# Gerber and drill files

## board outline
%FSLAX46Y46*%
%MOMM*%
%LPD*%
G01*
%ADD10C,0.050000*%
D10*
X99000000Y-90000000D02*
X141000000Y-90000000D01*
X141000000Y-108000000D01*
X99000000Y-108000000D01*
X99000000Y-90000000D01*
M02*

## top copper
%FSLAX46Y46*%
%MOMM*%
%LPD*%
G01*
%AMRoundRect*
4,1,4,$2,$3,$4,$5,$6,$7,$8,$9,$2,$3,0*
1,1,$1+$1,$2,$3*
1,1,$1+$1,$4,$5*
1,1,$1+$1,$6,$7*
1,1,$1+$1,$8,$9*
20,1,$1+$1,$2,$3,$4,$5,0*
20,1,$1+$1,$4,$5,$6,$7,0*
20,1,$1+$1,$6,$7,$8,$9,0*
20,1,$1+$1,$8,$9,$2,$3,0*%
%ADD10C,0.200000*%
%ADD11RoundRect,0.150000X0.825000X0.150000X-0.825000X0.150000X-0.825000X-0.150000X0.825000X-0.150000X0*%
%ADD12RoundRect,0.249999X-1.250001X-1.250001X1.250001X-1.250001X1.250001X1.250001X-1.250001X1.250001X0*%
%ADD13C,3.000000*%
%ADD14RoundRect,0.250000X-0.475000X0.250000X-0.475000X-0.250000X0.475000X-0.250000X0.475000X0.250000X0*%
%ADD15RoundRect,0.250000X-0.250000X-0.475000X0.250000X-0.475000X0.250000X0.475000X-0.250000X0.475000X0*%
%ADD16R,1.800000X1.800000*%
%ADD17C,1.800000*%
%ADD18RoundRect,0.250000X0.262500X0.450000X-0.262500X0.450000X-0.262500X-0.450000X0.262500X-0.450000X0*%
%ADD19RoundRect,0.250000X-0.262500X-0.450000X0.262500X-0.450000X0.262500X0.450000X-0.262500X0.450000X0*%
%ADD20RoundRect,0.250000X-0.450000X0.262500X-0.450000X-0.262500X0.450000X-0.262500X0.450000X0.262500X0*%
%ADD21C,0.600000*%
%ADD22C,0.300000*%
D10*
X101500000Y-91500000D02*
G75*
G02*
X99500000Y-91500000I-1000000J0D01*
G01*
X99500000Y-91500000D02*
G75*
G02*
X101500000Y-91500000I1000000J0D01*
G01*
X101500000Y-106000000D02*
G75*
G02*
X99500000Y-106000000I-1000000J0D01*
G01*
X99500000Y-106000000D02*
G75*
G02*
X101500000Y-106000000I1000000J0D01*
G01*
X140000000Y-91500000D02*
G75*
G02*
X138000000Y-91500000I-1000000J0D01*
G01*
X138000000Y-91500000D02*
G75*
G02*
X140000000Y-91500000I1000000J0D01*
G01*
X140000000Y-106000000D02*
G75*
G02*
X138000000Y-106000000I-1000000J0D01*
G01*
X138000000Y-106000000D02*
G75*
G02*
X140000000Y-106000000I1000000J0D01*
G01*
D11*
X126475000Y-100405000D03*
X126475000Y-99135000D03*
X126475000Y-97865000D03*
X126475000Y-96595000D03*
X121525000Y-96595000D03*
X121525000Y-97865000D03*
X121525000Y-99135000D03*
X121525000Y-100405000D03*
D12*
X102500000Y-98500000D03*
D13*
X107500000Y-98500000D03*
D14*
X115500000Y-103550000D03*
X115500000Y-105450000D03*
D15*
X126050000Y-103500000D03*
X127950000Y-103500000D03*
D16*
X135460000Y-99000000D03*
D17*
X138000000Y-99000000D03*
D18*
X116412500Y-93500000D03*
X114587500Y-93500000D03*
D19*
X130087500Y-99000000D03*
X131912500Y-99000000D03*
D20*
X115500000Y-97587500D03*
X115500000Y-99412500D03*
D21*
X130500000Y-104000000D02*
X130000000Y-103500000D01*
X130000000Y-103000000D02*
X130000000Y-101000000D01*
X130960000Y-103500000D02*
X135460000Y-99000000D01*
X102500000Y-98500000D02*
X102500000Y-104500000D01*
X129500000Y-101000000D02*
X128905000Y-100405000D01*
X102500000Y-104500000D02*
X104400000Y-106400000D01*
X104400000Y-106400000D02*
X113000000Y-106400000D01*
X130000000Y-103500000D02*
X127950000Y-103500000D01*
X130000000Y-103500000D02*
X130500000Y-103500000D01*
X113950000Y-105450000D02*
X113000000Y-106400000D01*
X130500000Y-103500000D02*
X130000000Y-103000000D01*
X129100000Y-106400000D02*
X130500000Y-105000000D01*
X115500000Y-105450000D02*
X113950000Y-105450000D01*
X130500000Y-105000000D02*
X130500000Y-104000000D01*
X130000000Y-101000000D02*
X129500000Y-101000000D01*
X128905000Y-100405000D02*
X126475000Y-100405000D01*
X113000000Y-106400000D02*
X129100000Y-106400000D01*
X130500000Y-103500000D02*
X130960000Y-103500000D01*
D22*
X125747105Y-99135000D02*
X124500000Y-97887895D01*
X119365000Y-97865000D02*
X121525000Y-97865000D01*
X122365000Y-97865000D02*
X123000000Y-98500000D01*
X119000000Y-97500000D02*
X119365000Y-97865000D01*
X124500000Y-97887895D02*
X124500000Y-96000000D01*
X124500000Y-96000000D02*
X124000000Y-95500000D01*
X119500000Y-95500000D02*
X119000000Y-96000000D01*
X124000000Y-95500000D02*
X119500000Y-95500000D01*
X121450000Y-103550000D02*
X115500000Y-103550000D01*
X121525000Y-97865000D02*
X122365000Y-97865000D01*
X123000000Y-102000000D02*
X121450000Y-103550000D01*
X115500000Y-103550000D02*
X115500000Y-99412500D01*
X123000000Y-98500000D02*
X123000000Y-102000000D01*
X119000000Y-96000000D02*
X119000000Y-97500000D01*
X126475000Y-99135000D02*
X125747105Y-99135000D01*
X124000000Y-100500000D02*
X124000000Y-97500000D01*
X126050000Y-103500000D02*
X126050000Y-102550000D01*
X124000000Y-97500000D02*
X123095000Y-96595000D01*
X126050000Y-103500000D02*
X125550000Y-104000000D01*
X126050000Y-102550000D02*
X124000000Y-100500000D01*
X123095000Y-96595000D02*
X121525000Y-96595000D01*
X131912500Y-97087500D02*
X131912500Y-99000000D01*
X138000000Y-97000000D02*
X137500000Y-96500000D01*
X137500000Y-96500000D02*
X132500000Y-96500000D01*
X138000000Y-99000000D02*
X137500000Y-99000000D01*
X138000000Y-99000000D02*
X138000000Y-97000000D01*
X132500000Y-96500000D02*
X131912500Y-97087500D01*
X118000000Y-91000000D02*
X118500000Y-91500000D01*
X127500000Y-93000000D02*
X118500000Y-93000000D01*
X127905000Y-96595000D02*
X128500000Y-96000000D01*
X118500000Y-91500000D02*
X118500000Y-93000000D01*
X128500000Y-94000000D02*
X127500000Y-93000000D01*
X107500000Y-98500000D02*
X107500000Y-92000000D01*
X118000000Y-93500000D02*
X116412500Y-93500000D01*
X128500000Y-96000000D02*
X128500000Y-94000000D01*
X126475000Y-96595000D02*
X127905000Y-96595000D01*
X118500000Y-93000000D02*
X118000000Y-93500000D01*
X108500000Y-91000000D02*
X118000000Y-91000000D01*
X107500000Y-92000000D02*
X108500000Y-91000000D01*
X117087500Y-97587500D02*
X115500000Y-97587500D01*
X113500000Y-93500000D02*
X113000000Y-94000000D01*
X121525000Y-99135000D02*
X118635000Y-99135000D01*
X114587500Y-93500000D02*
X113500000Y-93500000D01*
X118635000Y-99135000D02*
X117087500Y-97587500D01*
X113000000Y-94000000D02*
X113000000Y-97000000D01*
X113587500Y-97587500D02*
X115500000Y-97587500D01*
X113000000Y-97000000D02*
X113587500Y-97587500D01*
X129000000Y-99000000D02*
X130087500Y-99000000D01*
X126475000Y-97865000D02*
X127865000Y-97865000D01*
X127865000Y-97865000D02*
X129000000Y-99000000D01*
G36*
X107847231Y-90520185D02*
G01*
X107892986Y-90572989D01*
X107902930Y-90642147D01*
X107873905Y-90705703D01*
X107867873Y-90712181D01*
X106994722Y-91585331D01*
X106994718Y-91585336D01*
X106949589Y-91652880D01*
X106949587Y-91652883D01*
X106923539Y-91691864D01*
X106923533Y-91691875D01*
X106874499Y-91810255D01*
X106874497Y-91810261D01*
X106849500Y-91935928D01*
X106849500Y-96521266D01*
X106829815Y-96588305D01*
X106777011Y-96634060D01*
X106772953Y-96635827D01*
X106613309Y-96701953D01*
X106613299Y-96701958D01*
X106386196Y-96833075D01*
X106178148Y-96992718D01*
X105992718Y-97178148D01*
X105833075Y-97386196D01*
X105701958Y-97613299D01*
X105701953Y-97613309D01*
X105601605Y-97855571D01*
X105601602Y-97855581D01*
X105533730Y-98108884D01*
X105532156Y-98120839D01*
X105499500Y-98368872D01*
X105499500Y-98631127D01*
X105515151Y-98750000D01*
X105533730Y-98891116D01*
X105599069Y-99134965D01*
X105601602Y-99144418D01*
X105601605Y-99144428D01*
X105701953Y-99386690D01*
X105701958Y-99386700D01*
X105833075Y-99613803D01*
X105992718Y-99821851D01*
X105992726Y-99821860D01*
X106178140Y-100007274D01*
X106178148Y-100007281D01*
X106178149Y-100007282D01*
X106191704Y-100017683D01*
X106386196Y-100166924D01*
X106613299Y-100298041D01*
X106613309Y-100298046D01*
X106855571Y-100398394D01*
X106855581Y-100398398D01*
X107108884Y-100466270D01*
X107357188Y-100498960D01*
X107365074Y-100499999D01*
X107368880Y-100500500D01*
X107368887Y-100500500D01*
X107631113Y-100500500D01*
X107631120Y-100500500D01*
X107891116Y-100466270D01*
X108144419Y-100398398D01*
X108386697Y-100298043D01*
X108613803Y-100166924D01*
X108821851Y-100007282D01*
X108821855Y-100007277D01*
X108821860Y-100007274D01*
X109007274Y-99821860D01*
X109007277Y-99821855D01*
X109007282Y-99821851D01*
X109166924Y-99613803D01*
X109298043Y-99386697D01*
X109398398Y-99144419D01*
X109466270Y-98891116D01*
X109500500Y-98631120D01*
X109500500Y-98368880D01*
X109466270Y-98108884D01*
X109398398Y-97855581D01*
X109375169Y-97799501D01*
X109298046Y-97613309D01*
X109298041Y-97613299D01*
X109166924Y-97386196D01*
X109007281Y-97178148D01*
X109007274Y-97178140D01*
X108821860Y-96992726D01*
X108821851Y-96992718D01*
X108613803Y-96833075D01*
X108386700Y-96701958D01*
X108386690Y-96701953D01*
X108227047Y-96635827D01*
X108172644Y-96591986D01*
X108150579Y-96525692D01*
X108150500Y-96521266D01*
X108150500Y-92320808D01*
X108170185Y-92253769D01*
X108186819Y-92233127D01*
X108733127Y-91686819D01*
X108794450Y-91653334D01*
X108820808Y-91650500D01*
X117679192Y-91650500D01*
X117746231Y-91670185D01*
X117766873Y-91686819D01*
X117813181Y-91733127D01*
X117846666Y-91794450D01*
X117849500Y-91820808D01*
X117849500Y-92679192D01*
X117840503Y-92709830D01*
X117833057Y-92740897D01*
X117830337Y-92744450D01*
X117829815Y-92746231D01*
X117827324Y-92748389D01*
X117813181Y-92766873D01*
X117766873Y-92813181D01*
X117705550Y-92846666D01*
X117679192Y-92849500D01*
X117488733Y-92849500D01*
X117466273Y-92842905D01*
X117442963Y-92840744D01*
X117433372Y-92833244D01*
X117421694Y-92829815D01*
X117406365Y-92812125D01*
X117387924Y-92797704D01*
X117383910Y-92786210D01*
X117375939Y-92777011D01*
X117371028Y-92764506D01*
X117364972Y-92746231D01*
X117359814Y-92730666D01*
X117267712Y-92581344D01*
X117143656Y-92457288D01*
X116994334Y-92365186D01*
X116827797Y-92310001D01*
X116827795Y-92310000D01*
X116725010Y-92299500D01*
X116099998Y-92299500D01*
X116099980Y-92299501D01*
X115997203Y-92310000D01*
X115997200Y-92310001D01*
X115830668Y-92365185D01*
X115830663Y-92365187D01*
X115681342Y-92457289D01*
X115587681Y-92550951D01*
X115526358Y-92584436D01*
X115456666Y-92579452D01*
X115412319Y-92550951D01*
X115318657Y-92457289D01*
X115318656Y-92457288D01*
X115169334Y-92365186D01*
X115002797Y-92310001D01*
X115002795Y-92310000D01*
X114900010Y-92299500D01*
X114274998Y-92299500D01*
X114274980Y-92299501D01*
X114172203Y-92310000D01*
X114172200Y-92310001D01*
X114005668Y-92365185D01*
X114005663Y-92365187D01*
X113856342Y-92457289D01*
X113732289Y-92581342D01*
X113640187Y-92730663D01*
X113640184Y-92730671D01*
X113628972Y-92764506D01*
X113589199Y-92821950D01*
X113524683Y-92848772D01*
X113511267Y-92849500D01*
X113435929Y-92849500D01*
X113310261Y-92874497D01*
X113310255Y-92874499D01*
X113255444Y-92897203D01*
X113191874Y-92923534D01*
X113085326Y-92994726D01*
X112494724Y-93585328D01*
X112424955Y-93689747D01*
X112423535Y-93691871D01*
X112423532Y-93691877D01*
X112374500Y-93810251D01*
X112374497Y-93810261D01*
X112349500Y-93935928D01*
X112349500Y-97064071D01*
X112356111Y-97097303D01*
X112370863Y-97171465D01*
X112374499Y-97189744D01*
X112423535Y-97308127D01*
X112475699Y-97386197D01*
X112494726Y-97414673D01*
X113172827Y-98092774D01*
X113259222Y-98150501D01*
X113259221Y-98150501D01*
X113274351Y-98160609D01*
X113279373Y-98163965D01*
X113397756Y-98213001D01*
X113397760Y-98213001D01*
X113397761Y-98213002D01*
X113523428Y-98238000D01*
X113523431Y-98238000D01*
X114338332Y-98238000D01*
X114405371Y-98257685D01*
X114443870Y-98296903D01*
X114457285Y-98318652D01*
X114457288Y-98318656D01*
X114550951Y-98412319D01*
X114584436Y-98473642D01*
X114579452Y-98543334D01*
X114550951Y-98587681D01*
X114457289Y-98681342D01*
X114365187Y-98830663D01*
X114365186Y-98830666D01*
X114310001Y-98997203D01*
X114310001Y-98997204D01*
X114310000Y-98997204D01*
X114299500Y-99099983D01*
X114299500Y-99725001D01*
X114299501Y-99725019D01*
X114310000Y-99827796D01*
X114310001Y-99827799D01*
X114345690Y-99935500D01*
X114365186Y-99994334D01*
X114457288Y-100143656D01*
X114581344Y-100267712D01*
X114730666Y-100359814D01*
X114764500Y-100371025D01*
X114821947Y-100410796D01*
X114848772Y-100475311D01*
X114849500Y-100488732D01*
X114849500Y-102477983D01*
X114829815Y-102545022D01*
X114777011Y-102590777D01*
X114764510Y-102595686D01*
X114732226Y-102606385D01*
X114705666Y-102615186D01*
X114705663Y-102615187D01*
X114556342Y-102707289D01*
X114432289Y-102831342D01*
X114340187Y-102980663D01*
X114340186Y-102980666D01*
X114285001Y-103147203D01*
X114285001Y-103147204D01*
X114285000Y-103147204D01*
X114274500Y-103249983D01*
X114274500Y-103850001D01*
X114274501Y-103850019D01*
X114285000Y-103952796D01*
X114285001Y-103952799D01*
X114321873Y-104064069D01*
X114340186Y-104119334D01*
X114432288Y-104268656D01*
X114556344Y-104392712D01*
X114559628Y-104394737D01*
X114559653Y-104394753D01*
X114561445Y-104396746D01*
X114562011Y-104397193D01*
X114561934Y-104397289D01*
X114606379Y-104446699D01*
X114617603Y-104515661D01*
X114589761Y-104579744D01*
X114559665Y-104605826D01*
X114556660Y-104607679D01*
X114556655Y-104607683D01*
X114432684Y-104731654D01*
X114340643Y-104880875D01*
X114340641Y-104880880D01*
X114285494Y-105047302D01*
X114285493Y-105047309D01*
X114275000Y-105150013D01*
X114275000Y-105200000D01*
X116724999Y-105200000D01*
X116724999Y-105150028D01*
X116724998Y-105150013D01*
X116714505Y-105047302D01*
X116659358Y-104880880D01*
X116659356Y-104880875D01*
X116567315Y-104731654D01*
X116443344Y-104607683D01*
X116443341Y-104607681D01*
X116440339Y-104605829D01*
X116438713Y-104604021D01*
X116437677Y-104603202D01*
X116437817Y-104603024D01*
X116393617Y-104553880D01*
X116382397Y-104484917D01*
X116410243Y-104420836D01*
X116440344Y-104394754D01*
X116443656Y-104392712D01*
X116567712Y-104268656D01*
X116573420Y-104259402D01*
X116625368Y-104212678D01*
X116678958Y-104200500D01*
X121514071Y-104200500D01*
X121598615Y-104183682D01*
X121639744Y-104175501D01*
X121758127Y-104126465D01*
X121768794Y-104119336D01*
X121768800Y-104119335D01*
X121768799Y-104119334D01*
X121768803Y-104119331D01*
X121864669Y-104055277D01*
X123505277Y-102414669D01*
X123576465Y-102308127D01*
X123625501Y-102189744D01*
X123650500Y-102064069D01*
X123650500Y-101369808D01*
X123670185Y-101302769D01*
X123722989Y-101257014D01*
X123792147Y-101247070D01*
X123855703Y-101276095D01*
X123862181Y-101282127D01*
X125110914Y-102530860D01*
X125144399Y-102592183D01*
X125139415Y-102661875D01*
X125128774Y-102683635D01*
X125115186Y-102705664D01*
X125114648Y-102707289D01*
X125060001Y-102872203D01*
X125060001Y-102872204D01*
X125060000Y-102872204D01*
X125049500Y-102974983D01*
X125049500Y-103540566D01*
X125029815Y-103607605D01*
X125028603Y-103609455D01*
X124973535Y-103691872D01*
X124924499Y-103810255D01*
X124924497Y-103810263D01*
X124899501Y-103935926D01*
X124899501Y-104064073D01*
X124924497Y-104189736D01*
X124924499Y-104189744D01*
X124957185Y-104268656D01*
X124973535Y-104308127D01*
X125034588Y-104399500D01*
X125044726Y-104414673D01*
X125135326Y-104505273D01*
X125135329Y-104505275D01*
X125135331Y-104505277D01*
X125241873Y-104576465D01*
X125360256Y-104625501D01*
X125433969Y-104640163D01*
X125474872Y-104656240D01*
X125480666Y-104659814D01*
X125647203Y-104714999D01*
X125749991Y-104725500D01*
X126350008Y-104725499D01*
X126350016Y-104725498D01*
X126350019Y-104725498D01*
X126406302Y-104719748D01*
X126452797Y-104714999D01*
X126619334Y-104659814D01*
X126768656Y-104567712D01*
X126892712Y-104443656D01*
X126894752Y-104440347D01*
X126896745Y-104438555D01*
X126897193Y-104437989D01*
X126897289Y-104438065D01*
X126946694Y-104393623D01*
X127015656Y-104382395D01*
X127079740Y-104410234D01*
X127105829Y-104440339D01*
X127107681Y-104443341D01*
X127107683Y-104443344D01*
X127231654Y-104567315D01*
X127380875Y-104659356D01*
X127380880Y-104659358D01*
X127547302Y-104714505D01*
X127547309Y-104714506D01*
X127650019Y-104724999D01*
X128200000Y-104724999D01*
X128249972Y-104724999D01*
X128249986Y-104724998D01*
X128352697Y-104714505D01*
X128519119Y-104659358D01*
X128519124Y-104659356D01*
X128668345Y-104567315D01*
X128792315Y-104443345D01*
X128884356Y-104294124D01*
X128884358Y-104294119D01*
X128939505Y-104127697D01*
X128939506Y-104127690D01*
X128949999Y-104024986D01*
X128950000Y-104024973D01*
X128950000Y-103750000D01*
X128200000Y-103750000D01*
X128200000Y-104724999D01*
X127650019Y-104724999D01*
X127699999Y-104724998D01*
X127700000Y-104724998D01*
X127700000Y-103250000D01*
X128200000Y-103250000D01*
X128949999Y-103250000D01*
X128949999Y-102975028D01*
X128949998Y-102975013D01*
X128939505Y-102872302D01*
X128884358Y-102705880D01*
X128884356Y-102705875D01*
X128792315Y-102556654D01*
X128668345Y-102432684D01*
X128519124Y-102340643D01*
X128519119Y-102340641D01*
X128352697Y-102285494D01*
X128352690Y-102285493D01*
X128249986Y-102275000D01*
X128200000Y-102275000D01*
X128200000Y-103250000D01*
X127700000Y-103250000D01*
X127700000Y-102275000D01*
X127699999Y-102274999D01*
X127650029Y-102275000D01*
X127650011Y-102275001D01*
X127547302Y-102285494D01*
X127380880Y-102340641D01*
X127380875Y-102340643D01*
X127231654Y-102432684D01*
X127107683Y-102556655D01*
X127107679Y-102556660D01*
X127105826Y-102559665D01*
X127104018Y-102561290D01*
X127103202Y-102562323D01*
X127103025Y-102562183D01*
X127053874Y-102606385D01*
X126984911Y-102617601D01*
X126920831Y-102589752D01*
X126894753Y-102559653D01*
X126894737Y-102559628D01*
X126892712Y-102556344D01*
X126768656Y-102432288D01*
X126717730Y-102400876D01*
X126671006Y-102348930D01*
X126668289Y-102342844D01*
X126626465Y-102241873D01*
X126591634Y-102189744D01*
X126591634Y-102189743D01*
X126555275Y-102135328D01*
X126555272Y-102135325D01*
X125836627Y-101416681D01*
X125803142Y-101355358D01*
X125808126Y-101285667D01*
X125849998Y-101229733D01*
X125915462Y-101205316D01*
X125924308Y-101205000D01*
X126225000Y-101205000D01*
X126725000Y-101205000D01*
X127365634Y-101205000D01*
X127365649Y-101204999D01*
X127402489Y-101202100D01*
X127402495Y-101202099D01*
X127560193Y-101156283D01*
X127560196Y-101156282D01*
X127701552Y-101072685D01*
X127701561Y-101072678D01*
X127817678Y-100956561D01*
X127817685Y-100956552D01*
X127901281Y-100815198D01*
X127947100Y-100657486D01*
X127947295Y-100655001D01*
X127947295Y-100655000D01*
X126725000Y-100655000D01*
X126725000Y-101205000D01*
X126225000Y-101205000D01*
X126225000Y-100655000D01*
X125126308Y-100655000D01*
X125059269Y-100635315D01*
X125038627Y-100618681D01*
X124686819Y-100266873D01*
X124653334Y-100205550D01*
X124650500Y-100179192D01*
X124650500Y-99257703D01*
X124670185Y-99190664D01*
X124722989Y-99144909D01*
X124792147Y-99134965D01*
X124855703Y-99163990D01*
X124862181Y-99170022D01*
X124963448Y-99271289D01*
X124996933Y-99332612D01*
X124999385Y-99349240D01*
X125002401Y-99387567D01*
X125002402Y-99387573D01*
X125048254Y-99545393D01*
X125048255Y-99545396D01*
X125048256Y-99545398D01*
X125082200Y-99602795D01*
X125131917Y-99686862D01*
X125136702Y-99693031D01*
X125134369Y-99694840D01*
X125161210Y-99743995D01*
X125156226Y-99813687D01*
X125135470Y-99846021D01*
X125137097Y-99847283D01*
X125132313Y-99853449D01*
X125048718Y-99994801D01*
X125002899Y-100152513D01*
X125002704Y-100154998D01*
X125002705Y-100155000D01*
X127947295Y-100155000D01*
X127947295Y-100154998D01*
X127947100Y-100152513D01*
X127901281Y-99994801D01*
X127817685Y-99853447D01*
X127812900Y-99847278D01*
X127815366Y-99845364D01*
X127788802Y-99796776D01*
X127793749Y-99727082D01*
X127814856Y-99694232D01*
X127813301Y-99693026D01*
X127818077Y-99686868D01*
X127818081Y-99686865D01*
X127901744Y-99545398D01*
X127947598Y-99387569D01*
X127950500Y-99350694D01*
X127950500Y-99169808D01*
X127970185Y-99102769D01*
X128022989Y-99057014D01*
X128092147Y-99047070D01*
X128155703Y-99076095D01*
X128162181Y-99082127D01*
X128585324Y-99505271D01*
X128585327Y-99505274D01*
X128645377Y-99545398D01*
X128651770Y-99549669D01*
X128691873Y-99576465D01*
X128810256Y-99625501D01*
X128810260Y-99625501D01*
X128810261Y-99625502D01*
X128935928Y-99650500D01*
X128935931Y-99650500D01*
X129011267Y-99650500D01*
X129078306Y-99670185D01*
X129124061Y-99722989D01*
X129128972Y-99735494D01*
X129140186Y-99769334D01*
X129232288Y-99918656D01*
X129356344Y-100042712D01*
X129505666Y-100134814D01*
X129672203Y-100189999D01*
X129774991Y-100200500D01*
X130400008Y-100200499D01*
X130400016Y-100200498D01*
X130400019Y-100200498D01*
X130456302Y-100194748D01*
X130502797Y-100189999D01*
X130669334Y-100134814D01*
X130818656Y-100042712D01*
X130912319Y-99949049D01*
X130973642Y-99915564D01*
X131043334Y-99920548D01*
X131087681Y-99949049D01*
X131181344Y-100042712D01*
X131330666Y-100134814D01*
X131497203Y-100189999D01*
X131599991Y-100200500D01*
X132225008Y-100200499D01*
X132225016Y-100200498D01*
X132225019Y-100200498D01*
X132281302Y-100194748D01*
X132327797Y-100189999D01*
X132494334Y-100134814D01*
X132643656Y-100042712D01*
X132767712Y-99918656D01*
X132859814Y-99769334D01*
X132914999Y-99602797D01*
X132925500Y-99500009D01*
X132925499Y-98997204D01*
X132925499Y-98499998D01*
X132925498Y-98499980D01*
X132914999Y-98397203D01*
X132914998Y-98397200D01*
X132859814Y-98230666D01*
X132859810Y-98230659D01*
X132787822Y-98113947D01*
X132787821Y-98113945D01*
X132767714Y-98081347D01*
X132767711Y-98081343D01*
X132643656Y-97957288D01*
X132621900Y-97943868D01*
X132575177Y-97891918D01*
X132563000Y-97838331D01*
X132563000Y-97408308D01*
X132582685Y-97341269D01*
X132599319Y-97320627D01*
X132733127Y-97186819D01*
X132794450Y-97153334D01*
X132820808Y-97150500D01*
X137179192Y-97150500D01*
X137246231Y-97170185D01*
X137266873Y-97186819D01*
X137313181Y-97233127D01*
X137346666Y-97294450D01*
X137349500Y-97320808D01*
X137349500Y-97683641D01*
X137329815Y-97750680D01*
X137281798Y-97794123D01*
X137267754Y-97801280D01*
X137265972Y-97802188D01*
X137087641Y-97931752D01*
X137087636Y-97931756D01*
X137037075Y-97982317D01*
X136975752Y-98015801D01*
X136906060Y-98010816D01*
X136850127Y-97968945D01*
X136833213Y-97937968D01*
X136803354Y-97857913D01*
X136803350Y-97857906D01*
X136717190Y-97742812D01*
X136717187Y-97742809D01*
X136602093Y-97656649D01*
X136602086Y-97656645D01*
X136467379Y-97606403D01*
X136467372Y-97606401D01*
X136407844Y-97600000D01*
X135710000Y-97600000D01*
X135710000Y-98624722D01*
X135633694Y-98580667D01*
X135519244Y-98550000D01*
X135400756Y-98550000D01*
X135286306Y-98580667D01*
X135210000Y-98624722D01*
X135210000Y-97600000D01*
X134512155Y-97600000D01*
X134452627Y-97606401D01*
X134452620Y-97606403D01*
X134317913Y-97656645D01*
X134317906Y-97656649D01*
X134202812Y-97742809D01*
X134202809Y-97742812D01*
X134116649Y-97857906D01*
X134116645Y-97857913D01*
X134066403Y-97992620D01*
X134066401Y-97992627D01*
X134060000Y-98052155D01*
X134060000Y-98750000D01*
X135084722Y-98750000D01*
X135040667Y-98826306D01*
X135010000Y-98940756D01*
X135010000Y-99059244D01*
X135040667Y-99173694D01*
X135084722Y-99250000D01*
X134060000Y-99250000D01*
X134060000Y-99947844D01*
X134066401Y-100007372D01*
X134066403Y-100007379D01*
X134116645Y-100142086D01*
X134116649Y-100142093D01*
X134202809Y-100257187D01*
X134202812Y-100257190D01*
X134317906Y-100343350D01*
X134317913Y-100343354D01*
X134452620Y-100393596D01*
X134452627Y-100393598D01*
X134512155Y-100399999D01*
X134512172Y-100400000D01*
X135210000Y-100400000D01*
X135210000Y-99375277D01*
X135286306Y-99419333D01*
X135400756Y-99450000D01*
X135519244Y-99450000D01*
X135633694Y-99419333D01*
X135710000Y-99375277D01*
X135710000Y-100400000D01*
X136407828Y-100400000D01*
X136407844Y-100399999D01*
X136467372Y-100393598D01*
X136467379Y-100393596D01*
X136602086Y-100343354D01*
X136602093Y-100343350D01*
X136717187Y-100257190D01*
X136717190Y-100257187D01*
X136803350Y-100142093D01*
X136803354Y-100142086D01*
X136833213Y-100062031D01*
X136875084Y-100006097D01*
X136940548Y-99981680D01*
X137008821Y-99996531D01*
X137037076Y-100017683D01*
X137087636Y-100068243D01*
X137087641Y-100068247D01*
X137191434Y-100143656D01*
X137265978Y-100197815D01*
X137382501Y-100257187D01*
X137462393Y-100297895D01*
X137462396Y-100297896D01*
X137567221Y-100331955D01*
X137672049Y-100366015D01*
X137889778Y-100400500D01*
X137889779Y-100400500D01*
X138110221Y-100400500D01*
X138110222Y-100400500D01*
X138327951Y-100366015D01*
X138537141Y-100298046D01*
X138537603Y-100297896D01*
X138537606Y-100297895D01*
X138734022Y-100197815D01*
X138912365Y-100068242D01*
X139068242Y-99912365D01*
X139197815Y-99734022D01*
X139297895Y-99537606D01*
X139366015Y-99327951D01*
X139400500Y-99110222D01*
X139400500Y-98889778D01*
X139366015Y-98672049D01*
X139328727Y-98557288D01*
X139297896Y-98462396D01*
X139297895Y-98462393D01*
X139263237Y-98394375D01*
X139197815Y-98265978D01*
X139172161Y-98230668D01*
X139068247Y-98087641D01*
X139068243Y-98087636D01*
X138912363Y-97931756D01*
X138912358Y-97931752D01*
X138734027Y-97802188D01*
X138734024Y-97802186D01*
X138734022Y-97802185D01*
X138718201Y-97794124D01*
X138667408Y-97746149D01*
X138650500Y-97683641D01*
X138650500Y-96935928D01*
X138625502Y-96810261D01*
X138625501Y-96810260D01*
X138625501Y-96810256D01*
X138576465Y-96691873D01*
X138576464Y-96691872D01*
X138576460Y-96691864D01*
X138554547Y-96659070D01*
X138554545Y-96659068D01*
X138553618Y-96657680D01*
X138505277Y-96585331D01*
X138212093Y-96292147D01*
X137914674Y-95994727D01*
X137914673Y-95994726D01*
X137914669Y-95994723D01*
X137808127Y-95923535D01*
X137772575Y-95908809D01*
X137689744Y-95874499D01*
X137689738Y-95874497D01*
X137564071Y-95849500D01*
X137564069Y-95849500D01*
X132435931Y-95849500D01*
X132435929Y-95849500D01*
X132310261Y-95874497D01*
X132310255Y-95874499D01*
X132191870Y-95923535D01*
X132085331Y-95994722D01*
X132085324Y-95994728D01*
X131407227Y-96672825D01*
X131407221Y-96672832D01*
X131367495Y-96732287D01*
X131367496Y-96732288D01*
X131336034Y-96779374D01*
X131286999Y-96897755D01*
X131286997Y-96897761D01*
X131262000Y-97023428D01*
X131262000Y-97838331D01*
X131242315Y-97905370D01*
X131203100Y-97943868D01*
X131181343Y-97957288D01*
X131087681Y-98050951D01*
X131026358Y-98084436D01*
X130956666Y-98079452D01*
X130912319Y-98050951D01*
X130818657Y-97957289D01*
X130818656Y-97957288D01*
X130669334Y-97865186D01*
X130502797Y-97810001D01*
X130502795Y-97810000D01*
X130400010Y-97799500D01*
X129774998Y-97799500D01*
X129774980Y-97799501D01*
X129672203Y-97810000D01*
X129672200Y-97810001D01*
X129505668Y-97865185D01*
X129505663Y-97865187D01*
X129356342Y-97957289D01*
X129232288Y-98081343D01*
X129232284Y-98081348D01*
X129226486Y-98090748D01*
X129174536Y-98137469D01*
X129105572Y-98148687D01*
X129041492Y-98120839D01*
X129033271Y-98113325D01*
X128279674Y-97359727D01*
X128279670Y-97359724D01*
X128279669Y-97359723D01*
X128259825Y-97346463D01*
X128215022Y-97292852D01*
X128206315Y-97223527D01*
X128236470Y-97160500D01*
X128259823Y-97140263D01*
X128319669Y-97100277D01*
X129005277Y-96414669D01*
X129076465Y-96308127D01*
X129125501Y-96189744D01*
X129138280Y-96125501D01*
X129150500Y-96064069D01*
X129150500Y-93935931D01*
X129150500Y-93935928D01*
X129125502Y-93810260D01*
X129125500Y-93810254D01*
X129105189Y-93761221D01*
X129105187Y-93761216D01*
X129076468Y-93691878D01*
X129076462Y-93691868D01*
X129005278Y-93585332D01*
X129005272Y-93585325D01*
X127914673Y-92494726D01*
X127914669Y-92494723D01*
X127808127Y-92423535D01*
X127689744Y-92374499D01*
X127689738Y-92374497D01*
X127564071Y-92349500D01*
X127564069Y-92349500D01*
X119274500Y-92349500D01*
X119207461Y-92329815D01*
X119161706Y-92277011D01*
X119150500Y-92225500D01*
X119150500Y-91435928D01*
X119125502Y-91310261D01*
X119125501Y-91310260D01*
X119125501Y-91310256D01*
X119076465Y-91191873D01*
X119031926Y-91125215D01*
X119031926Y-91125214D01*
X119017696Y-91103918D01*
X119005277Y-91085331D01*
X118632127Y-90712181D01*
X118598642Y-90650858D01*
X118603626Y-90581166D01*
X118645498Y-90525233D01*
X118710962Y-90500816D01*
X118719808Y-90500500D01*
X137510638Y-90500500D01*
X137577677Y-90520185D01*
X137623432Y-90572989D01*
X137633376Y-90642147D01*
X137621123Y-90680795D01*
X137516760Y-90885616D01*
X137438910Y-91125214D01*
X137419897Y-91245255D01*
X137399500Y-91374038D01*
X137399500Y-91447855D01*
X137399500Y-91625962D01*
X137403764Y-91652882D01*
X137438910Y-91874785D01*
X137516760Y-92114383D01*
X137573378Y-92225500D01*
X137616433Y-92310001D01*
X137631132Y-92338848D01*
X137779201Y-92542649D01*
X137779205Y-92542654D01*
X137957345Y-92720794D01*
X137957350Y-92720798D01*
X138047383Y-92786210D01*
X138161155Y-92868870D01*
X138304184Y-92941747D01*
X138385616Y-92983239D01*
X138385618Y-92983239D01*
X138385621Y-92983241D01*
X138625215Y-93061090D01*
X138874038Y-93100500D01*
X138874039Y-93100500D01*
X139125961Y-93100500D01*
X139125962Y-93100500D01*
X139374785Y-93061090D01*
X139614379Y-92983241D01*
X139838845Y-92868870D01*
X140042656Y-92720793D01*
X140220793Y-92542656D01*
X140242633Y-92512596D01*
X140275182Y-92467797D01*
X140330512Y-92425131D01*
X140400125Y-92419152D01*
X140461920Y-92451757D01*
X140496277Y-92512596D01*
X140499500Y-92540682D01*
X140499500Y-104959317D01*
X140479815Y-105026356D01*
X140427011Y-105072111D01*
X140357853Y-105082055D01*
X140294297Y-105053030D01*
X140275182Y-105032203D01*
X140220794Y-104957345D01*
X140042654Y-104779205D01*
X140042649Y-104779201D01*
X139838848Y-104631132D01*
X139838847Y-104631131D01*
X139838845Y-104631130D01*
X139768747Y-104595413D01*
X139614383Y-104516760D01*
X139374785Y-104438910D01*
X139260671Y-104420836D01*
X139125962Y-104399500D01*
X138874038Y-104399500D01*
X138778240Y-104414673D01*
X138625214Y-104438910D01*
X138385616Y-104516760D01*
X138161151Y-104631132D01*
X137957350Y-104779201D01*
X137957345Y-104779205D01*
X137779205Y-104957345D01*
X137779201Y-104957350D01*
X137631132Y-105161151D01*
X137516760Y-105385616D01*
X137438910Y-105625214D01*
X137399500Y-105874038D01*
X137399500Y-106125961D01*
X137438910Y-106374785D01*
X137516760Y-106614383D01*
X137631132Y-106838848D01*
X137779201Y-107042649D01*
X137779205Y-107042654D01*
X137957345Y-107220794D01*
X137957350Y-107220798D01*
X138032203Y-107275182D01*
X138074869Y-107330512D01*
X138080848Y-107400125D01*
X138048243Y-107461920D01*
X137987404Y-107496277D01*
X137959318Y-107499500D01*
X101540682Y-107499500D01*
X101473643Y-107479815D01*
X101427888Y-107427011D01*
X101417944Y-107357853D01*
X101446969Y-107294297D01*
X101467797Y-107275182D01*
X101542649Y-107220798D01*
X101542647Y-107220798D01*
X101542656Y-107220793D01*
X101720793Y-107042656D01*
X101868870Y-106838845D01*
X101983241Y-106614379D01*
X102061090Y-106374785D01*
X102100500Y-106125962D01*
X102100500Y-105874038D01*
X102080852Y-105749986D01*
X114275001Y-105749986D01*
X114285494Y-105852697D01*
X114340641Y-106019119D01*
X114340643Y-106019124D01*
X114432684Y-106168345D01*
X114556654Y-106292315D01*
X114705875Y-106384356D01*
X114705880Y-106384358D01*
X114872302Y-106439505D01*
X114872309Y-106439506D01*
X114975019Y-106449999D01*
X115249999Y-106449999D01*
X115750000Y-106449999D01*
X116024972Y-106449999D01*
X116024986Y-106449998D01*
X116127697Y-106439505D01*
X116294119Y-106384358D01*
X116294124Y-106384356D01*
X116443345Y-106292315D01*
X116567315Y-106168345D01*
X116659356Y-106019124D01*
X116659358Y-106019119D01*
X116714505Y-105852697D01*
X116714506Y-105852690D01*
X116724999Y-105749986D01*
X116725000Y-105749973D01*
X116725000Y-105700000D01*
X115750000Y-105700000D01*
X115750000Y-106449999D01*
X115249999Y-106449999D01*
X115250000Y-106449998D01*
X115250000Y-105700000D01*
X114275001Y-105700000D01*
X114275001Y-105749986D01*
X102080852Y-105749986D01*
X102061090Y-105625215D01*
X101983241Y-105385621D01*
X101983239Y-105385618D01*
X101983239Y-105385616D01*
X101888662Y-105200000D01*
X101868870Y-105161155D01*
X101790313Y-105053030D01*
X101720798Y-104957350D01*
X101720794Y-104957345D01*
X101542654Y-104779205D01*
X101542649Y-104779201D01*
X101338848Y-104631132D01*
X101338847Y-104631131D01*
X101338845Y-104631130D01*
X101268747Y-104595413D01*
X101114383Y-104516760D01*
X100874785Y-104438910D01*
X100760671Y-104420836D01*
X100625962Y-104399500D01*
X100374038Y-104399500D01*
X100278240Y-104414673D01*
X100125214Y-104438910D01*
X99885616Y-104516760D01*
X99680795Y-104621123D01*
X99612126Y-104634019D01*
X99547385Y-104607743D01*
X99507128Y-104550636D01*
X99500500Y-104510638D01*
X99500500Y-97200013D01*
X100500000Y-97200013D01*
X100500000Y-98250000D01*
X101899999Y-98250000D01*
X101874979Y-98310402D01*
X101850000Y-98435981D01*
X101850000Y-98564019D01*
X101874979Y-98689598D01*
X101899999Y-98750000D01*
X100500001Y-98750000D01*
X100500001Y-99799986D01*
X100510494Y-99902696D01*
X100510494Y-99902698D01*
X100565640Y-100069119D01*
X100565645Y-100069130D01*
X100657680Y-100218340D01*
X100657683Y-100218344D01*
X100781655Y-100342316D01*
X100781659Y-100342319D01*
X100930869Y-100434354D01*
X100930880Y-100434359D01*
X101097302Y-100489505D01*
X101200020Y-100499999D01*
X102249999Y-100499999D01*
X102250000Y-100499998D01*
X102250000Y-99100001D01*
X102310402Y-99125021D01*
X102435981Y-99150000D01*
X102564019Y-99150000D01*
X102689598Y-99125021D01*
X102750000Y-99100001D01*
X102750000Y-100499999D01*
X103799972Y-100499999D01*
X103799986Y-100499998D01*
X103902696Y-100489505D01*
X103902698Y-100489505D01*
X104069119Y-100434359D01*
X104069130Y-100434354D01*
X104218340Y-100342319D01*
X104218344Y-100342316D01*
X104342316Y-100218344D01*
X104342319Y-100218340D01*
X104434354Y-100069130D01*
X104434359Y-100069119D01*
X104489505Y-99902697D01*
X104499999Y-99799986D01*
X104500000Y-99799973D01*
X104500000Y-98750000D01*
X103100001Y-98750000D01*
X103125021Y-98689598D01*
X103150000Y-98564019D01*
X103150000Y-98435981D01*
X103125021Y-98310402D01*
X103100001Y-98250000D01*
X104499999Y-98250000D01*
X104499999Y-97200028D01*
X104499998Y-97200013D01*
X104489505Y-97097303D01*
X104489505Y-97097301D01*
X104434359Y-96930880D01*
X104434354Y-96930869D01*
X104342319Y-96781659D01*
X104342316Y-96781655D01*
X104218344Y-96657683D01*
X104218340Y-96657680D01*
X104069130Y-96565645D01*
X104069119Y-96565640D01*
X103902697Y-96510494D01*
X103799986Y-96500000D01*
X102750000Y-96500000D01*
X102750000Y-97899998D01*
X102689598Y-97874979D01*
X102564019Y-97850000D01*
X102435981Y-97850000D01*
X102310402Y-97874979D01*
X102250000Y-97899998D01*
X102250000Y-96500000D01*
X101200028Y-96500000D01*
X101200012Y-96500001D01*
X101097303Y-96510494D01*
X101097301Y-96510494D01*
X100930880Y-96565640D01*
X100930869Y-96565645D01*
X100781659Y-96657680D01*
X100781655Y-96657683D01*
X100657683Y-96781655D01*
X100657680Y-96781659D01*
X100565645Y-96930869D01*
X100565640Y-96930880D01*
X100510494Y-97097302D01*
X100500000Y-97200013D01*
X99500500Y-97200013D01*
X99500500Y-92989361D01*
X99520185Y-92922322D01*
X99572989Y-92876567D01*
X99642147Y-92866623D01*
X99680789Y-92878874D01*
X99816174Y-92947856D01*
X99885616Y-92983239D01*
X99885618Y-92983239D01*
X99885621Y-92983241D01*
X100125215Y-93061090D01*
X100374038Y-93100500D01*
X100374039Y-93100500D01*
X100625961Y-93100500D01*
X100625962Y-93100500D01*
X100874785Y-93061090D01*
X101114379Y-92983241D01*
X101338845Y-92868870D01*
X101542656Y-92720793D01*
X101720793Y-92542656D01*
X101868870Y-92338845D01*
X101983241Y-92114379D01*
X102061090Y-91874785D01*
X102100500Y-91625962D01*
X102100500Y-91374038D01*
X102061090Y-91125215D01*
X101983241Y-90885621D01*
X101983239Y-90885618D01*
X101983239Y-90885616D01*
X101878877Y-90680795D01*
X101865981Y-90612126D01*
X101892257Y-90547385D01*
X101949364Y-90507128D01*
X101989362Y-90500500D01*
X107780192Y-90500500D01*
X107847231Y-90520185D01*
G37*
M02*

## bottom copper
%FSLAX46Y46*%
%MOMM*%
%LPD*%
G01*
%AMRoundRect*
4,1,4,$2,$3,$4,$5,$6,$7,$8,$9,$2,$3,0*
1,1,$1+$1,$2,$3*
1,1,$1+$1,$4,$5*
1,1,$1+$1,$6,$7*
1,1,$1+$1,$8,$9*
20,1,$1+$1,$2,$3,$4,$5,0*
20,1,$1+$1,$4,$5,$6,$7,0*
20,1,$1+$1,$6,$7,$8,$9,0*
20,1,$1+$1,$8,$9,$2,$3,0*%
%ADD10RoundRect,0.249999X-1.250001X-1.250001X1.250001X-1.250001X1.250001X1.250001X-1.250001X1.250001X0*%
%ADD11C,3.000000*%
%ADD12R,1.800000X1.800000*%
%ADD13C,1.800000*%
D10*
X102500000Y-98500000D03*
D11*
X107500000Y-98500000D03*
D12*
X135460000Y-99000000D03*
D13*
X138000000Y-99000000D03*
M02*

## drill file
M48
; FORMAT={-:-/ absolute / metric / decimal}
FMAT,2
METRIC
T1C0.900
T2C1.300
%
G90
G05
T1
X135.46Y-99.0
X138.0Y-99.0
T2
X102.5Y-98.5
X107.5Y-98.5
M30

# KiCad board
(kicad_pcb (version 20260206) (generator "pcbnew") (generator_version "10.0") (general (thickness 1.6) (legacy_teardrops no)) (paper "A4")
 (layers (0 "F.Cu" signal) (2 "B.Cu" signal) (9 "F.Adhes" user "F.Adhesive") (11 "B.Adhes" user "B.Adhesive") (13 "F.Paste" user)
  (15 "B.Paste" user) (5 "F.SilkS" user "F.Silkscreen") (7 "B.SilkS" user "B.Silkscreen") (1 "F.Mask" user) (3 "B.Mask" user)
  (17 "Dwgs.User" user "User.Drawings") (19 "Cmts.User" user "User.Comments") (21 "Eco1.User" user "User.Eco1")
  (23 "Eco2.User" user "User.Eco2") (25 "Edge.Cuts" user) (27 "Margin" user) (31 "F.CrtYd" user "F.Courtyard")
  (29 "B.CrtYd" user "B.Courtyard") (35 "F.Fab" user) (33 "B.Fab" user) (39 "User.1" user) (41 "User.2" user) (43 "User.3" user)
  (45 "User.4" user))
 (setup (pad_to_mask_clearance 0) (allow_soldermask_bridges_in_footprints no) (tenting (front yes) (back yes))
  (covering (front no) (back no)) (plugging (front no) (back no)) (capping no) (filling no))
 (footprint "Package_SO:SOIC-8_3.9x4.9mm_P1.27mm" (layer "F.Cu") (at 124 98.5 180)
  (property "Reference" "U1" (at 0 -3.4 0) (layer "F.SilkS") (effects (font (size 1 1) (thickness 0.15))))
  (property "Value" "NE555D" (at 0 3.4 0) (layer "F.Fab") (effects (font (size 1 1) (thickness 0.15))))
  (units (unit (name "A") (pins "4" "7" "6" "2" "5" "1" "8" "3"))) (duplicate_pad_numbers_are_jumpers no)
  (pad "1" smd roundrect (at -2.475 -1.905 180) (size 1.95 0.6) (layers "F.Cu" "F.Mask" "F.Paste") (roundrect_rratio 0.25) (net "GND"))
  (pad "2" smd roundrect (at -2.475 -0.635 180) (size 1.95 0.6) (layers "F.Cu" "F.Mask" "F.Paste") (roundrect_rratio 0.25)
   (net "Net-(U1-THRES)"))
  (pad "3" smd roundrect (at -2.475 0.635 180) (size 1.95 0.6) (layers "F.Cu" "F.Mask" "F.Paste") (roundrect_rratio 0.25)
   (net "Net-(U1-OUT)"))
  (pad "4" smd roundrect (at -2.475 1.905 180) (size 1.95 0.6) (layers "F.Cu" "F.Mask" "F.Paste") (roundrect_rratio 0.25)
   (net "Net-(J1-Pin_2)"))
  (pad "5" smd roundrect (at 2.475 1.905 180) (size 1.95 0.6) (layers "F.Cu" "F.Mask" "F.Paste") (roundrect_rratio 0.25)
   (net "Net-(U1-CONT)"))
  (pad "6" smd roundrect (at 2.475 0.635 180) (size 1.95 0.6) (layers "F.Cu" "F.Mask" "F.Paste") (roundrect_rratio 0.25)
   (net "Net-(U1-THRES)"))
  (pad "7" smd roundrect (at 2.475 -0.635 180) (size 1.95 0.6) (layers "F.Cu" "F.Mask" "F.Paste") (roundrect_rratio 0.25)
   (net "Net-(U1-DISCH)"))
  (pad "8" smd roundrect (at 2.475 -1.905 180) (size 1.95 0.6) (layers "F.Cu" "F.Mask" "F.Paste") (roundrect_rratio 0.25) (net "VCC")))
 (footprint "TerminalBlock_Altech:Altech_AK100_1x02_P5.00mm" (layer "F.Cu") (at 102.5 98.5)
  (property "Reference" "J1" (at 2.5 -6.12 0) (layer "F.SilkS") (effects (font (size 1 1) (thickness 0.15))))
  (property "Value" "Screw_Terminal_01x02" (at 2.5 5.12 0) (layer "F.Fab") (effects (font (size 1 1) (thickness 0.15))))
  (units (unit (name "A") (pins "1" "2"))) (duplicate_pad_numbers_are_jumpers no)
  (pad "1" thru_hole roundrect (at 0 0) (size 3 3) (drill 1.3) (layers "*.Cu" "*.Mask") (remove_unused_layers no)
   (roundrect_rratio 0.083333) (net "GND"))
  (pad "2" thru_hole circle (at 5 0) (size 3 3) (drill 1.3) (layers "*.Cu" "*.Mask") (remove_unused_layers no) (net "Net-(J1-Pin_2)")))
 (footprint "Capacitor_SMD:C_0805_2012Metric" (layer "F.Cu") (at 115.5 104.5 -90)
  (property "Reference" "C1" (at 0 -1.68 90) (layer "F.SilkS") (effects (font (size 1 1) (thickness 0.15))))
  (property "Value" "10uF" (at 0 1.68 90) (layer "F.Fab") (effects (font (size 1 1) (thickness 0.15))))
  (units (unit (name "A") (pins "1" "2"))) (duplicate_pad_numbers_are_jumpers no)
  (pad "1" smd roundrect (at -0.95 0 270) (size 1 1.45) (layers "F.Cu" "F.Mask" "F.Paste") (roundrect_rratio 0.25) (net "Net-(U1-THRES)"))
  (pad "2" smd roundrect (at 0.95 0 270) (size 1 1.45) (layers "F.Cu" "F.Mask" "F.Paste") (roundrect_rratio 0.25) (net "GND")))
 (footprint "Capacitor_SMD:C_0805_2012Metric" (layer "F.Cu") (at 127 103.5)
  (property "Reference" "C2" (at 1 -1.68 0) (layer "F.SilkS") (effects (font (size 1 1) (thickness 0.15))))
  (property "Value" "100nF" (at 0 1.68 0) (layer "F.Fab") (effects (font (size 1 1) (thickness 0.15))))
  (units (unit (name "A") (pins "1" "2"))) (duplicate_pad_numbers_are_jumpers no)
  (pad "1" smd roundrect (at -0.95 0) (size 1 1.45) (layers "F.Cu" "F.Mask" "F.Paste") (roundrect_rratio 0.25) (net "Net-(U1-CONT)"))
  (pad "2" smd roundrect (at 0.95 0) (size 1 1.45) (layers "F.Cu" "F.Mask" "F.Paste") (roundrect_rratio 0.25) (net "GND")))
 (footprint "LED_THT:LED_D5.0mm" (layer "F.Cu") (at 135.46 99)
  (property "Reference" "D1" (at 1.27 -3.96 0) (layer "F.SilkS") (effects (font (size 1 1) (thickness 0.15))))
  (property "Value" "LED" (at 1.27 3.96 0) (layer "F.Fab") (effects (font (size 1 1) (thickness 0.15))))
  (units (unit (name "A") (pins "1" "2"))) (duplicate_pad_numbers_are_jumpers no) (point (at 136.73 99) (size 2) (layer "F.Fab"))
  (pad "1" thru_hole rect (at 0 0) (size 1.8 1.8) (drill 0.9) (layers "*.Cu" "*.Mask") (remove_unused_layers no) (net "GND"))
  (pad "2" thru_hole circle (at 2.54 0) (size 1.8 1.8) (drill 0.9) (layers "*.Cu" "*.Mask") (remove_unused_layers no) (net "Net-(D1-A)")))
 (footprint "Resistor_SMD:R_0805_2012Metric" (layer "F.Cu") (at 115.5 93.5 180)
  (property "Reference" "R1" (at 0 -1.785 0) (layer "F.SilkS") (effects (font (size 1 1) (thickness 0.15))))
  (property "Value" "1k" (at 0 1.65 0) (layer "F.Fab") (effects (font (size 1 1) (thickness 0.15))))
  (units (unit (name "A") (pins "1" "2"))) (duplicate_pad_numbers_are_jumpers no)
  (pad "1" smd roundrect (at -0.9125 0 180) (size 1.025 1.4) (layers "F.Cu" "F.Mask" "F.Paste") (roundrect_rratio 0.243902)
   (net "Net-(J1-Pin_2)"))
  (pad "2" smd roundrect (at 0.9125 0 180) (size 1.025 1.4) (layers "F.Cu" "F.Mask" "F.Paste") (roundrect_rratio 0.243902)
   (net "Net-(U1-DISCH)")))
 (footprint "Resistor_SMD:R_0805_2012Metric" (layer "F.Cu") (at 131 99)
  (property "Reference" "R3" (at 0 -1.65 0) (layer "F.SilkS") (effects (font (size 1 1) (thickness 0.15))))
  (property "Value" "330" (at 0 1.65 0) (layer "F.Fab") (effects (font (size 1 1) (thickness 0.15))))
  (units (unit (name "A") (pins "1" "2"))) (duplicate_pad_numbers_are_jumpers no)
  (pad "1" smd roundrect (at -0.9125 0) (size 1.025 1.4) (layers "F.Cu" "F.Mask" "F.Paste") (roundrect_rratio 0.243902) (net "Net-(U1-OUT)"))
  (pad "2" smd roundrect (at 0.9125 0) (size 1.025 1.4) (layers "F.Cu" "F.Mask" "F.Paste") (roundrect_rratio 0.243902) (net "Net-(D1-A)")))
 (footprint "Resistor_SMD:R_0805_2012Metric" (layer "F.Cu") (at 115.5 98.5 -90)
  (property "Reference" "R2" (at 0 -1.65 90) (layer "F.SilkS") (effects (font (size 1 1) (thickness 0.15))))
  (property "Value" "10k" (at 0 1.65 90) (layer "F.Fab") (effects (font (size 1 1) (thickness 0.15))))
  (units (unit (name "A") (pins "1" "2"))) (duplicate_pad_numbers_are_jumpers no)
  (pad "1" smd roundrect (at -0.9125 0 270) (size 1.025 1.4) (layers "F.Cu" "F.Mask" "F.Paste") (roundrect_rratio 0.243902)
   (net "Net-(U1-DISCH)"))
  (pad "2" smd roundrect (at 0.9125 0 270) (size 1.025 1.4) (layers "F.Cu" "F.Mask" "F.Paste") (roundrect_rratio 0.243902)
   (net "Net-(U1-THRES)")))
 (gr_circle (center 100.5 91.5) (end 99.5 91.5) (stroke (width 0.2) (type default)) (fill no) (layer "F.Cu"))
 (gr_circle (center 100.5 106) (end 99.5 106) (stroke (width 0.2) (type default)) (fill no) (layer "F.Cu"))
 (gr_circle (center 139 91.5) (end 138 91.5) (stroke (width 0.2) (type default)) (fill no) (layer "F.Cu"))
 (gr_circle (center 139 106) (end 138 106) (stroke (width 0.2) (type default)) (fill no) (layer "F.Cu"))
 (gr_rect (start 99 90) (end 141 108) (stroke (width 0.05) (type default)) (fill no) (layer "Edge.Cuts"))
 (segment (start 130.5 104) (end 130 103.5) (width 0.6) (layer "F.Cu") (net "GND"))
 (segment (start 130 103) (end 130 101) (width 0.6) (layer "F.Cu") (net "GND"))
 (segment (start 130.96 103.5) (end 135.46 99) (width 0.6) (layer "F.Cu") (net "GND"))
 (segment (start 102.5 98.5) (end 102.5 104.5) (width 0.6) (layer "F.Cu") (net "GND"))
 (segment (start 129.5 101) (end 128.905 100.405) (width 0.6) (layer "F.Cu") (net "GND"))
 (segment (start 102.5 104.5) (end 104.4 106.4) (width 0.6) (layer "F.Cu") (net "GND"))
 (segment (start 104.4 106.4) (end 113 106.4) (width 0.6) (layer "F.Cu") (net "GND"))
 (segment (start 130 103.5) (end 127.95 103.5) (width 0.6) (layer "F.Cu") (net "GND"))
 (segment (start 130 103.5) (end 130.5 103.5) (width 0.6) (layer "F.Cu") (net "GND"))
 (segment (start 113.95 105.45) (end 113 106.4) (width 0.6) (layer "F.Cu") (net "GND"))
 (segment (start 130.5 103.5) (end 130 103) (width 0.6) (layer "F.Cu") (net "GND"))
 (segment (start 129.1 106.4) (end 130.5 105) (width 0.6) (layer "F.Cu") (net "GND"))
 (segment (start 115.5 105.45) (end 113.95 105.45) (width 0.6) (layer "F.Cu") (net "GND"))
 (segment (start 130.5 105) (end 130.5 104) (width 0.6) (layer "F.Cu") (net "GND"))
 (segment (start 130 101) (end 129.5 101) (width 0.6) (layer "F.Cu") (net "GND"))
 (segment (start 128.905 100.405) (end 126.475 100.405) (width 0.6) (layer "F.Cu") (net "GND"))
 (segment (start 113 106.4) (end 129.1 106.4) (width 0.6) (layer "F.Cu") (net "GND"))
 (segment (start 130.5 103.5) (end 130.96 103.5) (width 0.6) (layer "F.Cu") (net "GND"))
 (segment (start 125.747105 99.135) (end 124.5 97.887895) (width 0.3) (layer "F.Cu") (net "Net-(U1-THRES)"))
 (segment (start 119.365 97.865) (end 121.525 97.865) (width 0.3) (layer "F.Cu") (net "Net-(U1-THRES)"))
 (segment (start 122.365 97.865) (end 123 98.5) (width 0.3) (layer "F.Cu") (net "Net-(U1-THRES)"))
 (segment (start 119 97.5) (end 119.365 97.865) (width 0.3) (layer "F.Cu") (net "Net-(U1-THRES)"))
 (segment (start 124.5 97.887895) (end 124.5 96) (width 0.3) (layer "F.Cu") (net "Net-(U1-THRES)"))
 (segment (start 124.5 96) (end 124 95.5) (width 0.3) (layer "F.Cu") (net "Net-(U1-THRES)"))
 (segment (start 119.5 95.5) (end 119 96) (width 0.3) (layer "F.Cu") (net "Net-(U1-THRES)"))
 (segment (start 124 95.5) (end 119.5 95.5) (width 0.3) (layer "F.Cu") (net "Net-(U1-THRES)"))
 (segment (start 121.45 103.55) (end 115.5 103.55) (width 0.3) (layer "F.Cu") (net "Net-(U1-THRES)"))
 (segment (start 121.525 97.865) (end 122.365 97.865) (width 0.3) (layer "F.Cu") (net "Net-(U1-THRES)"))
 (segment (start 123 102) (end 121.45 103.55) (width 0.3) (layer "F.Cu") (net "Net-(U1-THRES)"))
 (segment (start 115.5 103.55) (end 115.5 99.4125) (width 0.3) (layer "F.Cu") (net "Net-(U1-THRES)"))
 (segment (start 123 98.5) (end 123 102) (width 0.3) (layer "F.Cu") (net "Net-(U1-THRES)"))
 (segment (start 119 96) (end 119 97.5) (width 0.3) (layer "F.Cu") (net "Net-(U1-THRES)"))
 (segment (start 126.475 99.135) (end 125.747105 99.135) (width 0.3) (layer "F.Cu") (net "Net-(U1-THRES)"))
 (segment (start 124 100.5) (end 124 97.5) (width 0.3) (layer "F.Cu") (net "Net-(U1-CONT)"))
 (segment (start 126.05 103.5) (end 126.05 102.55) (width 0.3) (layer "F.Cu") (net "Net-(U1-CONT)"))
 (segment (start 124 97.5) (end 123.095 96.595) (width 0.3) (layer "F.Cu") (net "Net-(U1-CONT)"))
 (segment (start 126.05 103.5) (end 125.55 104) (width 0.3) (layer "F.Cu") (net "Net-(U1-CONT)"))
 (segment (start 126.05 102.55) (end 124 100.5) (width 0.3) (layer "F.Cu") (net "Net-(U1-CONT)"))
 (segment (start 123.095 96.595) (end 121.525 96.595) (width 0.3) (layer "F.Cu") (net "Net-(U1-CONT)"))
 (segment (start 131.9125 97.0875) (end 131.9125 99) (width 0.3) (layer "F.Cu") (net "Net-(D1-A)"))
 (segment (start 138 97) (end 137.5 96.5) (width 0.3) (layer "F.Cu") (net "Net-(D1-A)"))
 (segment (start 137.5 96.5) (end 132.5 96.5) (width 0.3) (layer "F.Cu") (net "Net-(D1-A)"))
 (segment (start 138 99) (end 137.5 99) (width 0.3) (layer "F.Cu") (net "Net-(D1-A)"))
 (segment (start 138 99) (end 138 97) (width 0.3) (layer "F.Cu") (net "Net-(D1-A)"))
 (segment (start 132.5 96.5) (end 131.9125 97.0875) (width 0.3) (layer "F.Cu") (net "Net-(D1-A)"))
 (segment (start 118 91) (end 118.5 91.5) (width 0.3) (layer "F.Cu") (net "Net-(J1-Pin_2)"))
 (segment (start 127.5 93) (end 118.5 93) (width 0.3) (layer "F.Cu") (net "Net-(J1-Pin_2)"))
 (segment (start 127.905 96.595) (end 128.5 96) (width 0.3) (layer "F.Cu") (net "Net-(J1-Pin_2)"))
 (segment (start 118.5 91.5) (end 118.5 93) (width 0.3) (layer "F.Cu") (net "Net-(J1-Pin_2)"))
 (segment (start 128.5 94) (end 127.5 93) (width 0.3) (layer "F.Cu") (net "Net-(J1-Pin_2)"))
 (segment (start 107.5 98.5) (end 107.5 92) (width 0.3) (layer "F.Cu") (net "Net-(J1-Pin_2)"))
 (segment (start 118 93.5) (end 116.4125 93.5) (width 0.3) (layer "F.Cu") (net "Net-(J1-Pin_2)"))
 (segment (start 128.5 96) (end 128.5 94) (width 0.3) (layer "F.Cu") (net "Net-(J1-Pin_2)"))
 (segment (start 126.475 96.595) (end 127.905 96.595) (width 0.3) (layer "F.Cu") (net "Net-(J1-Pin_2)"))
 (segment (start 118.5 93) (end 118 93.5) (width 0.3) (layer "F.Cu") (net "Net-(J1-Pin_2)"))
 (segment (start 108.5 91) (end 118 91) (width 0.3) (layer "F.Cu") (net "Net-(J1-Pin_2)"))
 (segment (start 107.5 92) (end 108.5 91) (width 0.3) (layer "F.Cu") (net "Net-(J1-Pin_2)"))
 (segment (start 117.0875 97.5875) (end 115.5 97.5875) (width 0.3) (layer "F.Cu") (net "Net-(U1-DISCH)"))
 (segment (start 113.5 93.5) (end 113 94) (width 0.3) (layer "F.Cu") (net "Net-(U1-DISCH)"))
 (segment (start 121.525 99.135) (end 118.635 99.135) (width 0.3) (layer "F.Cu") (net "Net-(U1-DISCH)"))
 (segment (start 114.5875 93.5) (end 113.5 93.5) (width 0.3) (layer "F.Cu") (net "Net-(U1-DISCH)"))
 (segment (start 118.635 99.135) (end 117.0875 97.5875) (width 0.3) (layer "F.Cu") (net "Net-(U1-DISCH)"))
 (segment (start 113 94) (end 113 97) (width 0.3) (layer "F.Cu") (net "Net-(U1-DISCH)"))
 (segment (start 113.5875 97.5875) (end 115.5 97.5875) (width 0.3) (layer "F.Cu") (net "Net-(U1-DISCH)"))
 (segment (start 113 97) (end 113.5875 97.5875) (width 0.3) (layer "F.Cu") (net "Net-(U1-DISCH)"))
 (segment (start 129 99) (end 130.0875 99) (width 0.3) (layer "F.Cu") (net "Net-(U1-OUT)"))
 (segment (start 126.475 97.865) (end 127.865 97.865) (width 0.3) (layer "F.Cu") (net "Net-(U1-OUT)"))
 (segment (start 127.865 97.865) (end 129 99) (width 0.3) (layer "F.Cu") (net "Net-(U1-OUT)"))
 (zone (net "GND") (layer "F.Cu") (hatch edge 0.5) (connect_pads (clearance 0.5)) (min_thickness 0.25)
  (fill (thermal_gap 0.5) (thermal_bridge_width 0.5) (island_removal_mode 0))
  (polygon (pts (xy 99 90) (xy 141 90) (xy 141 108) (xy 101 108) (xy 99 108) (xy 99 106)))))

